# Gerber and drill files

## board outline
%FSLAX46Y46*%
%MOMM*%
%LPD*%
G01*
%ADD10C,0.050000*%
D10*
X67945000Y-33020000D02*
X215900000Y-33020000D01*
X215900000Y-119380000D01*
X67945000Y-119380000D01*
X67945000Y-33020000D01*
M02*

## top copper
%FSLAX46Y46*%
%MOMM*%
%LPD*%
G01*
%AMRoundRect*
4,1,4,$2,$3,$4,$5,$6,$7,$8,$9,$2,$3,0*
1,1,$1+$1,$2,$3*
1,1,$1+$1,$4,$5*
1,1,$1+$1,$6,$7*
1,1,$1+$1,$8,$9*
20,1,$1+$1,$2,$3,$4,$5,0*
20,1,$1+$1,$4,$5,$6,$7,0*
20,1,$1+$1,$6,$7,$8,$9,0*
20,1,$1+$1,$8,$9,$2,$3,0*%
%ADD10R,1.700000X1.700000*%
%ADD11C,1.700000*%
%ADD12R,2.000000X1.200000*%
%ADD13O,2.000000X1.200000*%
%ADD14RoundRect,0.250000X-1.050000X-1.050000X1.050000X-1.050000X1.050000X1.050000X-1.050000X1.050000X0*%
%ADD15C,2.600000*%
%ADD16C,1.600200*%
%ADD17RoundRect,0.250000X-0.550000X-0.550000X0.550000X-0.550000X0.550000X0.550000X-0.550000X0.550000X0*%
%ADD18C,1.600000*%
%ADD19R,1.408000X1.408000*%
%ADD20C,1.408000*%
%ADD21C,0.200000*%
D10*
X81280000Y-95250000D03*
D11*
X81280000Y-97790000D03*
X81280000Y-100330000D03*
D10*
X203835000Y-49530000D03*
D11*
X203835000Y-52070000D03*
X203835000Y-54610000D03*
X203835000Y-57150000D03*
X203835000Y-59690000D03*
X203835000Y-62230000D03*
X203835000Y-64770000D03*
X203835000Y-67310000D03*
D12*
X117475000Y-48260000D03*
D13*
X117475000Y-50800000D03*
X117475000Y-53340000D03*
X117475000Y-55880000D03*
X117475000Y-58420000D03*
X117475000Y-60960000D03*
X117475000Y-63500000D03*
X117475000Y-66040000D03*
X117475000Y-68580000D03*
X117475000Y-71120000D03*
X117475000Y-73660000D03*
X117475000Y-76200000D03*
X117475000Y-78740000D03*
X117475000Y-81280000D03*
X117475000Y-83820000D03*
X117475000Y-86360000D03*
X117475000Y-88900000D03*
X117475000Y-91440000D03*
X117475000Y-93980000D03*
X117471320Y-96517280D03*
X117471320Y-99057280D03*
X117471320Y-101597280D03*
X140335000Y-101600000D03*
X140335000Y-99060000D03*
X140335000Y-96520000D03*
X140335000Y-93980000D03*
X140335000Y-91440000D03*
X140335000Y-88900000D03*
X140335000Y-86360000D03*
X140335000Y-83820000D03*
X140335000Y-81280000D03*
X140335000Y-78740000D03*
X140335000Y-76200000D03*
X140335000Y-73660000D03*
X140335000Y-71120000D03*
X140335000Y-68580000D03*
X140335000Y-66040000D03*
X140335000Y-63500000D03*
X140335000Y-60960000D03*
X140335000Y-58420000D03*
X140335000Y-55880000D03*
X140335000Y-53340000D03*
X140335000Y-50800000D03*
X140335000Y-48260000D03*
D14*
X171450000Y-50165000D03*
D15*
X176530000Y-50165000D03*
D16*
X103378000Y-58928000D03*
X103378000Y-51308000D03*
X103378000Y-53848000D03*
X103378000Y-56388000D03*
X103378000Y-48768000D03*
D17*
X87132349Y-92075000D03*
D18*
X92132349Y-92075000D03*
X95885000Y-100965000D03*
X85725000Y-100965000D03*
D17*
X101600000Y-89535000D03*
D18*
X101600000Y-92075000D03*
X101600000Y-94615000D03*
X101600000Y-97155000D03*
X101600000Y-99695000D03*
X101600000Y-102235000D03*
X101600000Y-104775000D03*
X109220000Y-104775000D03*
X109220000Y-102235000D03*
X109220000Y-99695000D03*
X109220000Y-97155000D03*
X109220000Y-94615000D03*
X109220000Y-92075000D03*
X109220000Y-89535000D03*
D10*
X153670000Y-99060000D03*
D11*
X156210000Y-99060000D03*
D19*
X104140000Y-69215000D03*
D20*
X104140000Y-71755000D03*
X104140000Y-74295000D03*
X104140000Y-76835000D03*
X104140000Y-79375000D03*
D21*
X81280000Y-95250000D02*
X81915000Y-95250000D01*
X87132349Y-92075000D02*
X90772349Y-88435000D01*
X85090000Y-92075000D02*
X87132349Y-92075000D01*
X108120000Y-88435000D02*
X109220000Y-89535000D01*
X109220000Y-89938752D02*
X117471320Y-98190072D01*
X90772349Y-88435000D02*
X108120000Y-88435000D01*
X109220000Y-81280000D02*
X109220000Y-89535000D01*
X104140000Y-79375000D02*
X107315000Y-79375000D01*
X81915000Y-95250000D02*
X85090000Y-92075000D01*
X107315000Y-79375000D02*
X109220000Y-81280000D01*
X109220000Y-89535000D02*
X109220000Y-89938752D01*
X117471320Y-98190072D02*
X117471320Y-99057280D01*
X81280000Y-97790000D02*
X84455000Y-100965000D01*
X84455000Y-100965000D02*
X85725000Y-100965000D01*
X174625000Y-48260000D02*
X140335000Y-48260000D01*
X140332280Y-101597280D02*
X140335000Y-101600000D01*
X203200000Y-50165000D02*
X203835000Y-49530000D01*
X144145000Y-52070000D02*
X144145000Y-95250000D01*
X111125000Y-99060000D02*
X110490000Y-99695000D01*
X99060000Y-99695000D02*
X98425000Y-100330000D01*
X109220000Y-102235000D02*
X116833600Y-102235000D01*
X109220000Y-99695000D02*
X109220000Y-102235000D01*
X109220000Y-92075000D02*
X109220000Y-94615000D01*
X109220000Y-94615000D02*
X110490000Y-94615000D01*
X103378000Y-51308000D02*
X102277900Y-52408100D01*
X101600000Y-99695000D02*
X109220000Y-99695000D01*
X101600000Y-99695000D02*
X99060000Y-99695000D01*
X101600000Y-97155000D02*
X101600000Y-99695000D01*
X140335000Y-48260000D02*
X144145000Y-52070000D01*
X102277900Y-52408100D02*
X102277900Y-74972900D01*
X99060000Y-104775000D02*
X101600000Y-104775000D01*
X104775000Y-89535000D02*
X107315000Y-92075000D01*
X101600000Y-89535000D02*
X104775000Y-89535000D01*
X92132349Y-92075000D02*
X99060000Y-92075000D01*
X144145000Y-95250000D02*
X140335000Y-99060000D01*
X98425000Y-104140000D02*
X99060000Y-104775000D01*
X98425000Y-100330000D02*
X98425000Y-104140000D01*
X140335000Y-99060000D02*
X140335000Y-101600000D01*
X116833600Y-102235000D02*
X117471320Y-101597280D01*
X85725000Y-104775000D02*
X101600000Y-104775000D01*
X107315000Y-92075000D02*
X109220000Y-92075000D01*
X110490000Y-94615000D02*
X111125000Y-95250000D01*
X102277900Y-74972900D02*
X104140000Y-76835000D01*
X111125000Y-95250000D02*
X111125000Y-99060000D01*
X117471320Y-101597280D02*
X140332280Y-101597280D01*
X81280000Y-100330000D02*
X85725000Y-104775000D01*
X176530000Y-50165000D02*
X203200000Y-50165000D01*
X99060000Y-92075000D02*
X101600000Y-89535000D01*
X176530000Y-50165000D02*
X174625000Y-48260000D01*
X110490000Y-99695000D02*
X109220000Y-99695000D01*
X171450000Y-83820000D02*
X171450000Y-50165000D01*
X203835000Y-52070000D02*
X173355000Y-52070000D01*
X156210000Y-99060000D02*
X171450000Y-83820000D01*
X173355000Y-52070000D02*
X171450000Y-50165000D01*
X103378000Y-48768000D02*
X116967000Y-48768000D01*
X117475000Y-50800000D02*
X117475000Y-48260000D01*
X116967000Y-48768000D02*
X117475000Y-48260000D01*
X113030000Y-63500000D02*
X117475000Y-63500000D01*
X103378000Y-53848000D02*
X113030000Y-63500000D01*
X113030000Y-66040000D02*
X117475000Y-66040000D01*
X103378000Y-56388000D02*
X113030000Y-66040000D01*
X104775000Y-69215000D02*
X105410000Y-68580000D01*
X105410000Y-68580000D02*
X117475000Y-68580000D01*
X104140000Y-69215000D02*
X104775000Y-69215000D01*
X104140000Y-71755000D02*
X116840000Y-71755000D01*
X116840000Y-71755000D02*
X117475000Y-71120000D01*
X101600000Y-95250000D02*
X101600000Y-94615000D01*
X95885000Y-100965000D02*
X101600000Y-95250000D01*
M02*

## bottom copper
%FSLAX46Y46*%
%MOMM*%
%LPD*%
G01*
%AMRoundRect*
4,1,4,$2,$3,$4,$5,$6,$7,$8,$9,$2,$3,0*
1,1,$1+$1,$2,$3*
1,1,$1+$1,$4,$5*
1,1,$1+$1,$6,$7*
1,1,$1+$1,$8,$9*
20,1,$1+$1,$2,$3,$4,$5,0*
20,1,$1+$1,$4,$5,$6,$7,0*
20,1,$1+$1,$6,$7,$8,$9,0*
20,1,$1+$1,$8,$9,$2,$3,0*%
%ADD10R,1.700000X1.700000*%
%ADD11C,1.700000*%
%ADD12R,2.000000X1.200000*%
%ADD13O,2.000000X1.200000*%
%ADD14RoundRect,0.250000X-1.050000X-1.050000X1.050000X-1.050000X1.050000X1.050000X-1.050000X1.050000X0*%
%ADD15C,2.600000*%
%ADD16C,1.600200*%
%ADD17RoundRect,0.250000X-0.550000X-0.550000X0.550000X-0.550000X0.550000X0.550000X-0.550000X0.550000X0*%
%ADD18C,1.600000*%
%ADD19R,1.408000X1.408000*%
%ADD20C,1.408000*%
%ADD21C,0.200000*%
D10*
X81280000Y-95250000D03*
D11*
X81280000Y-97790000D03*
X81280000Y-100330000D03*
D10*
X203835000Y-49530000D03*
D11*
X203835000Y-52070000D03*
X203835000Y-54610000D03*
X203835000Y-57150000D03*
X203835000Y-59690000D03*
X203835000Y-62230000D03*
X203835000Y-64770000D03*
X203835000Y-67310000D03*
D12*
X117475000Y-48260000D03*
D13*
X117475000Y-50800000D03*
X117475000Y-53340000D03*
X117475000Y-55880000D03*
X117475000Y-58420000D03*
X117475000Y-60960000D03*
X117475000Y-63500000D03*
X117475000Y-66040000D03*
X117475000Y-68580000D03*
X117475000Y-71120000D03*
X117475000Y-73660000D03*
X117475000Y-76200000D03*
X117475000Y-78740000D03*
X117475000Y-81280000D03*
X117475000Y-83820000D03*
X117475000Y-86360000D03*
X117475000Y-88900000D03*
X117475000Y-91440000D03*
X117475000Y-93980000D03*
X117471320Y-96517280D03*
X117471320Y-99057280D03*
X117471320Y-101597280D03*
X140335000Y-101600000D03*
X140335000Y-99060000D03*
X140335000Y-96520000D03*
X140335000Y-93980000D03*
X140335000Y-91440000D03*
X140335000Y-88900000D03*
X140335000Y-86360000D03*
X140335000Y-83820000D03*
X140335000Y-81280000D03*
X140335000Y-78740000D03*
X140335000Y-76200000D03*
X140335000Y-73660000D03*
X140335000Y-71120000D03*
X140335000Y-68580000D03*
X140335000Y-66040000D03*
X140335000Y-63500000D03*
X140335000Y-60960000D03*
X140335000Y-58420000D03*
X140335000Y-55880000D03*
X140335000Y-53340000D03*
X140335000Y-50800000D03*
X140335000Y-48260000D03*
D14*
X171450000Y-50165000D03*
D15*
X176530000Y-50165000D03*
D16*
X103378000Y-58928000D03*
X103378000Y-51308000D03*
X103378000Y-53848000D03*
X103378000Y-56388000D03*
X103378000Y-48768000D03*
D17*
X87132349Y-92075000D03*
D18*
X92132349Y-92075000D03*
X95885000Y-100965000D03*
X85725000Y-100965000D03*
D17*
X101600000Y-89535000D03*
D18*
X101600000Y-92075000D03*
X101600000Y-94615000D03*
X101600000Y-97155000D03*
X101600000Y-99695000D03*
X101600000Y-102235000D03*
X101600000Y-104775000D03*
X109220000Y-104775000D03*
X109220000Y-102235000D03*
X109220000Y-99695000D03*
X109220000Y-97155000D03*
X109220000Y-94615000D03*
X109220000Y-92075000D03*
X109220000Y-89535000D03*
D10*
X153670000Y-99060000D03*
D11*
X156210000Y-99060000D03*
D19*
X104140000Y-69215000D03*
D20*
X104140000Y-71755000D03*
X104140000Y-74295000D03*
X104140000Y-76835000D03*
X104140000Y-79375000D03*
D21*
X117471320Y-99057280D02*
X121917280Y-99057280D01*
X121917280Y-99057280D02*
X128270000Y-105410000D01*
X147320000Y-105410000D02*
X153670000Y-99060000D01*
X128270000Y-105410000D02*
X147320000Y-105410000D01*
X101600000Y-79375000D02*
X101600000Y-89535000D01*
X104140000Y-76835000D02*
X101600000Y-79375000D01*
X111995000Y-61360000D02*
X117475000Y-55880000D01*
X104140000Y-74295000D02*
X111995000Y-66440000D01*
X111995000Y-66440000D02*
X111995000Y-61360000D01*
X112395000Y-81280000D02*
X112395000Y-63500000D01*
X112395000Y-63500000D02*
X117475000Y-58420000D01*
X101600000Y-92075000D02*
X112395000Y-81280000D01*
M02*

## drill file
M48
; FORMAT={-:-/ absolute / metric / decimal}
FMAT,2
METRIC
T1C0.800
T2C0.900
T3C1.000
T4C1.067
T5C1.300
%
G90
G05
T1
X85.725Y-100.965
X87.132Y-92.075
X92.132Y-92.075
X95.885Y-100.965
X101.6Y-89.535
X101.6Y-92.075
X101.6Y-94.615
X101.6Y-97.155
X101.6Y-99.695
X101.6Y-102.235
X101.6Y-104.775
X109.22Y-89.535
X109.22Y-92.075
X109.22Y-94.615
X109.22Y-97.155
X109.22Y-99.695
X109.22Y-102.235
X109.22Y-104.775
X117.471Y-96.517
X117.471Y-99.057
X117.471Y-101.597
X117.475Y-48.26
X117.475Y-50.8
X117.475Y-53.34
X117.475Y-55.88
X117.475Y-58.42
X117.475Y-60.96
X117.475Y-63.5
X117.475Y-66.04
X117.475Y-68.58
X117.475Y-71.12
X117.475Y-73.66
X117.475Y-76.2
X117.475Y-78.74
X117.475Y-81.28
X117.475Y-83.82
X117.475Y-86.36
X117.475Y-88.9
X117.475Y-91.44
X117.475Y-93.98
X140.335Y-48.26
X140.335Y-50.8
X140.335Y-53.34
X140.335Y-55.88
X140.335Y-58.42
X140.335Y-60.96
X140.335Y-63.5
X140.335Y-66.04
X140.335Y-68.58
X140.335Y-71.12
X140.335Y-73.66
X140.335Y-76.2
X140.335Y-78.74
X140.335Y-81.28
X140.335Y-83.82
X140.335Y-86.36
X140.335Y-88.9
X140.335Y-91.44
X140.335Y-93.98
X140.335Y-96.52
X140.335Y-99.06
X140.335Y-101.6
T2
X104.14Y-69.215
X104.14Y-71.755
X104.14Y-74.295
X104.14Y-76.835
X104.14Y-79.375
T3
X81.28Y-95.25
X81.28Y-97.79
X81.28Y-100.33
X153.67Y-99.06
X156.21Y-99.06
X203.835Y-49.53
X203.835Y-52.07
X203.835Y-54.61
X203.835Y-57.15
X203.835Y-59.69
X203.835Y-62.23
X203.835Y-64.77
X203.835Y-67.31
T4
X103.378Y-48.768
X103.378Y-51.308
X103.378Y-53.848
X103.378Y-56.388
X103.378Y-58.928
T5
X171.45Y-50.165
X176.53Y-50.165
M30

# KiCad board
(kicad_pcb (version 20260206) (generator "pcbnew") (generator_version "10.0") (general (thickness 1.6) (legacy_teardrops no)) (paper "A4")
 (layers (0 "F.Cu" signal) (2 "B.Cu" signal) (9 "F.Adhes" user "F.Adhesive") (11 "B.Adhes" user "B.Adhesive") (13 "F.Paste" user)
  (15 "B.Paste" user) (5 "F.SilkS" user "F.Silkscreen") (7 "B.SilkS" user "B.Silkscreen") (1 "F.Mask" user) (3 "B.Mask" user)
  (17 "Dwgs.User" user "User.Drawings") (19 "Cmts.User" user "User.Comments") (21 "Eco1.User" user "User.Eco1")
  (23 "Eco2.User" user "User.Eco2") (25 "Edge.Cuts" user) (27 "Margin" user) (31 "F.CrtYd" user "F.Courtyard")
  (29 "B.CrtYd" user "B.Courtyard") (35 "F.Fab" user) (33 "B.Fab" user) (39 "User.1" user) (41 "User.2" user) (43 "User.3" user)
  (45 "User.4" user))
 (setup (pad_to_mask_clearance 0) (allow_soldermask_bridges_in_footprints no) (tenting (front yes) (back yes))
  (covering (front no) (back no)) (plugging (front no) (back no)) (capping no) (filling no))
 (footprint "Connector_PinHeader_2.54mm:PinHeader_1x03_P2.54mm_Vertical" (layer "F.Cu") (at 81.28 95.25)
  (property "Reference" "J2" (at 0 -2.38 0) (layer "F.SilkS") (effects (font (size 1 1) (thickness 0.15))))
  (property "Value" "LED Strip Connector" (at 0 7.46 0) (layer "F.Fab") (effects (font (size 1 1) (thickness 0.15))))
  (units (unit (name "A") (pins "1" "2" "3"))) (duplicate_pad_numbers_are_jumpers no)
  (pad "1" thru_hole rect (at 0 0) (size 1.7 1.7) (drill 1) (layers "*.Cu" "*.Mask") (remove_unused_layers no) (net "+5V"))
  (pad "2" thru_hole circle (at 0 2.54) (size 1.7 1.7) (drill 1) (layers "*.Cu" "*.Mask") (remove_unused_layers no) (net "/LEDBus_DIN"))
  (pad "3" thru_hole circle (at 0 5.08) (size 1.7 1.7) (drill 1) (layers "*.Cu" "*.Mask") (remove_unused_layers no) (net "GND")))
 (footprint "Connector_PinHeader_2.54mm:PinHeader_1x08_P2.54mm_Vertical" (layer "F.Cu") (at 203.835 49.53)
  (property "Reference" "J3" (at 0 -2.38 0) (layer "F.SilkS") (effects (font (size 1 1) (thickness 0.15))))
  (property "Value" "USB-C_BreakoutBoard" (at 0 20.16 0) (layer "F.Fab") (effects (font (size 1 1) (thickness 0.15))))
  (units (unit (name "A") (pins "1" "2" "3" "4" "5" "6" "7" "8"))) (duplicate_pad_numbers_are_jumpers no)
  (pad "1" thru_hole rect (at 0 0) (size 1.7 1.7) (drill 1) (layers "*.Cu" "*.Mask") (remove_unused_layers no) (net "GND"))
  (pad "2" thru_hole circle (at 0 2.54) (size 1.7 1.7) (drill 1) (layers "*.Cu" "*.Mask") (remove_unused_layers no) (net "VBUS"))
  (pad "3" thru_hole circle (at 0 5.08) (size 1.7 1.7) (drill 1) (layers "*.Cu" "*.Mask") (remove_unused_layers no)
   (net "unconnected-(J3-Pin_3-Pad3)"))
  (pad "4" thru_hole circle (at 0 7.62) (size 1.7 1.7) (drill 1) (layers "*.Cu" "*.Mask") (remove_unused_layers no)
   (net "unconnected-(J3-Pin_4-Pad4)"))
  (pad "5" thru_hole circle (at 0 10.16) (size 1.7 1.7) (drill 1) (layers "*.Cu" "*.Mask") (remove_unused_layers no)
   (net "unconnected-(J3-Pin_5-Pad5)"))
  (pad "6" thru_hole circle (at 0 12.7) (size 1.7 1.7) (drill 1) (layers "*.Cu" "*.Mask") (remove_unused_layers no)
   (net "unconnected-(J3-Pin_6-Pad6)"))
  (pad "7" thru_hole circle (at 0 15.24) (size 1.7 1.7) (drill 1) (layers "*.Cu" "*.Mask") (remove_unused_layers no)
   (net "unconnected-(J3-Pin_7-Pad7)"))
  (pad "8" thru_hole circle (at 0 17.78) (size 1.7 1.7) (drill 1) (layers "*.Cu" "*.Mask") (remove_unused_layers no)
   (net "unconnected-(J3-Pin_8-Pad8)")))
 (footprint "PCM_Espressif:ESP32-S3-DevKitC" (layer "F.Cu") (at 117.475 48.26)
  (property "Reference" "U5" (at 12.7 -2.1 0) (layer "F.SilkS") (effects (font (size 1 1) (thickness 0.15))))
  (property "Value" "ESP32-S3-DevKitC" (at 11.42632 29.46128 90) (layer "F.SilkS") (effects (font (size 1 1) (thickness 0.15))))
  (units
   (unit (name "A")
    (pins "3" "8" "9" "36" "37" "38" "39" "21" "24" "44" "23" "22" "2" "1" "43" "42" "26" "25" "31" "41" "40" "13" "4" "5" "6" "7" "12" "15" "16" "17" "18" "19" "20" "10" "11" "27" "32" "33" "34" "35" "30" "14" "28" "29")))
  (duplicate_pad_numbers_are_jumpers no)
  (pad "1" thru_hole rect (at 0 0 270) (size 1.2 2) (drill 0.8) (layers "*.Cu" "*.Mask") (remove_unused_layers no) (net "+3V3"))
  (pad "2" thru_hole oval (at 0 2.54 270) (size 1.2 2) (drill 0.8) (layers "*.Cu" "*.Mask") (remove_unused_layers no) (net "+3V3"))
  (pad "3" thru_hole oval (at 0 5.08 270) (size 1.2 2) (drill 0.8) (layers "*.Cu" "*.Mask") (remove_unused_layers no)
   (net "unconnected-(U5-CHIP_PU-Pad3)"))
  (pad "4" thru_hole oval (at 0 7.62 270) (size 1.2 2) (drill 0.8) (layers "*.Cu" "*.Mask") (remove_unused_layers no)
   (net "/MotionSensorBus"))
  (pad "5" thru_hole oval (at 0 10.16 270) (size 1.2 2) (drill 0.8) (layers "*.Cu" "*.Mask") (remove_unused_layers no) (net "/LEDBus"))
  (pad "6" thru_hole oval (at 0 12.7 270) (size 1.2 2) (drill 0.8) (layers "*.Cu" "*.Mask") (remove_unused_layers no)
   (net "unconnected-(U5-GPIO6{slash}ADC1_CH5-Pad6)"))
  (pad "7" thru_hole oval (at 0 15.24 270) (size 1.2 2) (drill 0.8) (layers "*.Cu" "*.Mask") (remove_unused_layers no) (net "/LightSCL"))
  (pad "8" thru_hole oval (at 0 17.78 270) (size 1.2 2) (drill 0.8) (layers "*.Cu" "*.Mask") (remove_unused_layers no) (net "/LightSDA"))
  (pad "9" thru_hole oval (at 0 20.32 270) (size 1.2 2) (drill 0.8) (layers "*.Cu" "*.Mask") (remove_unused_layers no)
   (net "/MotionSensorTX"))
  (pad "10" thru_hole oval (at 0 22.86 270) (size 1.2 2) (drill 0.8) (layers "*.Cu" "*.Mask") (remove_unused_layers no)
   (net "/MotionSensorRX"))
  (pad "11" thru_hole oval (at 0 25.4 270) (size 1.2 2) (drill 0.8) (layers "*.Cu" "*.Mask") (remove_unused_layers no)
   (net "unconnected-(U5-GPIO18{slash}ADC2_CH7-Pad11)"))
  (pad "12" thru_hole oval (at 0 27.94 270) (size 1.2 2) (drill 0.8) (layers "*.Cu" "*.Mask") (remove_unused_layers no)
   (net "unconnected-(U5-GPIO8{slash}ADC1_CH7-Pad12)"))
  (pad "13" thru_hole oval (at 0 30.48 270) (size 1.2 2) (drill 0.8) (layers "*.Cu" "*.Mask") (remove_unused_layers no)
   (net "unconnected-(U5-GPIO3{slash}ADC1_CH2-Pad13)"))
  (pad "14" thru_hole oval (at 0 33.02 270) (size 1.2 2) (drill 0.8) (layers "*.Cu" "*.Mask") (remove_unused_layers no)
   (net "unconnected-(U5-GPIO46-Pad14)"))
  (pad "15" thru_hole oval (at 0 35.56 270) (size 1.2 2) (drill 0.8) (layers "*.Cu" "*.Mask") (remove_unused_layers no)
   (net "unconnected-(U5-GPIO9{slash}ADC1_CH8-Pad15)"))
  (pad "16" thru_hole oval (at 0 38.1 270) (size 1.2 2) (drill 0.8) (layers "*.Cu" "*.Mask") (remove_unused_layers no)
   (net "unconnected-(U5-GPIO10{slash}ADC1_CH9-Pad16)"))
  (pad "17" thru_hole oval (at 0 40.64 270) (size 1.2 2) (drill 0.8) (layers "*.Cu" "*.Mask") (remove_unused_layers no)
   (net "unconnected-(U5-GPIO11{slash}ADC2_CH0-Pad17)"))
  (pad "18" thru_hole oval (at 0 43.18 270) (size 1.2 2) (drill 0.8) (layers "*.Cu" "*.Mask") (remove_unused_layers no)
   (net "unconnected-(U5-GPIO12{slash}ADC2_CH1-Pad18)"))
  (pad "19" thru_hole oval (at 0 45.72 270) (size 1.2 2) (drill 0.8) (layers "*.Cu" "*.Mask") (remove_unused_layers no)
   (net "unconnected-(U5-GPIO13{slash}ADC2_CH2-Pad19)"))
  (pad "20" thru_hole oval (at -0.00368 48.25728 270) (size 1.2 2) (drill 0.8) (layers "*.Cu" "*.Mask") (remove_unused_layers no)
   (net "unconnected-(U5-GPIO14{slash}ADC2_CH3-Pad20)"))
  (pad "21" thru_hole oval (at -0.00368 50.79728 270) (size 1.2 2) (drill 0.8) (layers "*.Cu" "*.Mask") (remove_unused_layers no)
   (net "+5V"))
  (pad "22" thru_hole oval (at -0.00368 53.33728 270) (size 1.2 2) (drill 0.8) (layers "*.Cu" "*.Mask") (remove_unused_layers no)
   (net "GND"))
  (pad "23" thru_hole oval (at 22.86 53.34 270) (size 1.2 2) (drill 0.8) (layers "*.Cu" "*.Mask") (remove_unused_layers no) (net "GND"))
  (pad "24" thru_hole oval (at 22.86 50.8 270) (size 1.2 2) (drill 0.8) (layers "*.Cu" "*.Mask") (remove_unused_layers no) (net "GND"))
  (pad "25" thru_hole oval (at 22.86 48.26 270) (size 1.2 2) (drill 0.8) (layers "*.Cu" "*.Mask") (remove_unused_layers no)
   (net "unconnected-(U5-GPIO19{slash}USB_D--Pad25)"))
  (pad "26" thru_hole oval (at 22.86 45.72 270) (size 1.2 2) (drill 0.8) (layers "*.Cu" "*.Mask") (remove_unused_layers no)
   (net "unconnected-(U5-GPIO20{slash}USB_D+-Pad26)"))
  (pad "27" thru_hole oval (at 22.86 43.18 270) (size 1.2 2) (drill 0.8) (layers "*.Cu" "*.Mask") (remove_unused_layers no)
   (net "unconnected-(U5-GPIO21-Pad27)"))
  (pad "28" thru_hole oval (at 22.86 40.64 270) (size 1.2 2) (drill 0.8) (layers "*.Cu" "*.Mask") (remove_unused_layers no)
   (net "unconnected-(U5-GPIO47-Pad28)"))
  (pad "29" thru_hole oval (at 22.86 38.1 270) (size 1.2 2) (drill 0.8) (layers "*.Cu" "*.Mask") (remove_unused_layers no)
   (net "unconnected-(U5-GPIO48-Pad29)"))
  (pad "30" thru_hole oval (at 22.86 35.56 270) (size 1.2 2) (drill 0.8) (layers "*.Cu" "*.Mask") (remove_unused_layers no)
   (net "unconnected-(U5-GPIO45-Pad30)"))
  (pad "31" thru_hole oval (at 22.86 33.02 270) (size 1.2 2) (drill 0.8) (layers "*.Cu" "*.Mask") (remove_unused_layers no)
   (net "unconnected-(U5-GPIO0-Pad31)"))
  (pad "32" thru_hole oval (at 22.86 30.48 270) (size 1.2 2) (drill 0.8) (layers "*.Cu" "*.Mask") (remove_unused_layers no)
   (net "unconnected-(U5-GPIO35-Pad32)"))
  (pad "33" thru_hole oval (at 22.86 27.94 270) (size 1.2 2) (drill 0.8) (layers "*.Cu" "*.Mask") (remove_unused_layers no)
   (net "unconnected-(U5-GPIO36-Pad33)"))
  (pad "34" thru_hole oval (at 22.86 25.4 270) (size 1.2 2) (drill 0.8) (layers "*.Cu" "*.Mask") (remove_unused_layers no)
   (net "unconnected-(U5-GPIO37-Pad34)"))
  (pad "35" thru_hole oval (at 22.86 22.86 270) (size 1.2 2) (drill 0.8) (layers "*.Cu" "*.Mask") (remove_unused_layers no)
   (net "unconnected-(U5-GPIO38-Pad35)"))
  (pad "36" thru_hole oval (at 22.86 20.32 270) (size 1.2 2) (drill 0.8) (layers "*.Cu" "*.Mask") (remove_unused_layers no)
   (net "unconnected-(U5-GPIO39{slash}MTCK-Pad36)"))
  (pad "37" thru_hole oval (at 22.86 17.78 270) (size 1.2 2) (drill 0.8) (layers "*.Cu" "*.Mask") (remove_unused_layers no)
   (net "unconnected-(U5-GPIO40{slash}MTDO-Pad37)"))
  (pad "38" thru_hole oval (at 22.86 15.24 270) (size 1.2 2) (drill 0.8) (layers "*.Cu" "*.Mask") (remove_unused_layers no)
   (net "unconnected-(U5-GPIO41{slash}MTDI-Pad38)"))
  (pad "39" thru_hole oval (at 22.86 12.7 270) (size 1.2 2) (drill 0.8) (layers "*.Cu" "*.Mask") (remove_unused_layers no)
   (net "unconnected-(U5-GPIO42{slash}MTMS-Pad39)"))
  (pad "40" thru_hole oval (at 22.86 10.16 270) (size 1.2 2) (drill 0.8) (layers "*.Cu" "*.Mask") (remove_unused_layers no)
   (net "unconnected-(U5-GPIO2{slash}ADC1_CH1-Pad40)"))
  (pad "41" thru_hole oval (at 22.86 7.62 270) (size 1.2 2) (drill 0.8) (layers "*.Cu" "*.Mask") (remove_unused_layers no)
   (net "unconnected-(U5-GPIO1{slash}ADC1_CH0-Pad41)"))
  (pad "42" thru_hole oval (at 22.86 5.08 270) (size 1.2 2) (drill 0.8) (layers "*.Cu" "*.Mask") (remove_unused_layers no)
   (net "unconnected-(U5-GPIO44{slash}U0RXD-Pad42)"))
  (pad "43" thru_hole oval (at 22.86 2.54 270) (size 1.2 2) (drill 0.8) (layers "*.Cu" "*.Mask") (remove_unused_layers no)
   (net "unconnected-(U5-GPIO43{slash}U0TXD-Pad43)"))
  (pad "44" thru_hole oval (at 22.86 0 270) (size 1.2 2) (drill 0.8) (layers "*.Cu" "*.Mask") (remove_unused_layers no) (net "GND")))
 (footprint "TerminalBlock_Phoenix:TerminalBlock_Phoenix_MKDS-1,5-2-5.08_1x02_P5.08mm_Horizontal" (layer "F.Cu") (at 171.45 50.165)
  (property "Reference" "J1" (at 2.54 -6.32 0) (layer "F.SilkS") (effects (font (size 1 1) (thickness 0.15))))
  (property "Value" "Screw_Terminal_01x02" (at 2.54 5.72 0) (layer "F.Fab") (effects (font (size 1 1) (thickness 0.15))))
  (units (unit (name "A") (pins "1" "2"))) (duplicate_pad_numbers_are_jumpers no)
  (pad "1" thru_hole roundrect (at 0 0) (size 2.6 2.6) (drill 1.3) (layers "*.Cu" "*.Mask") (remove_unused_layers no)
   (roundrect_rratio 0.096154) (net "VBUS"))
  (pad "2" thru_hole circle (at 5.08 0) (size 2.6 2.6) (drill 1.3) (layers "*.Cu" "*.Mask") (remove_unused_layers no) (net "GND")))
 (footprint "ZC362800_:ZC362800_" (layer "F.Cu") (at 102.108 53.848 -90)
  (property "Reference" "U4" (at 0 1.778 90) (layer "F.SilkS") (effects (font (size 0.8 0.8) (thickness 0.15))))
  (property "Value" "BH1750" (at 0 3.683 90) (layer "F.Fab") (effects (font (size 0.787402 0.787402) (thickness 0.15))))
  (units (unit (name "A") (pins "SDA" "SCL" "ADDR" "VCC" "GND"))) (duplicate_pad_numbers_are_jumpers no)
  (pad "ADDR" thru_hole circle (at 5.08 -1.27 270) (size 1.6002 1.6002) (drill 1.0668) (layers "*.Cu" "*.Mask") (remove_unused_layers no)
   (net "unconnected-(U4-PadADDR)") (solder_mask_margin 0.102))
  (pad "GND" thru_hole circle (at -2.54 -1.27 270) (size 1.6002 1.6002) (drill 1.0668) (layers "*.Cu" "*.Mask") (remove_unused_layers no)
   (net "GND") (solder_mask_margin 0.102))
  (pad "SCL" thru_hole circle (at 0 -1.27 270) (size 1.6002 1.6002) (drill 1.0668) (layers "*.Cu" "*.Mask") (remove_unused_layers no)
   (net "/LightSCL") (solder_mask_margin 0.102))
  (pad "SDA" thru_hole circle (at 2.54 -1.27 270) (size 1.6002 1.6002) (drill 1.0668) (layers "*.Cu" "*.Mask") (remove_unused_layers no)
   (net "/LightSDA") (solder_mask_margin 0.102))
  (pad "VCC" thru_hole circle (at -5.08 -1.27 270) (size 1.6002 1.6002) (drill 1.0668) (layers "*.Cu" "*.Mask") (remove_unused_layers no)
   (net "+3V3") (solder_mask_margin 0.102)))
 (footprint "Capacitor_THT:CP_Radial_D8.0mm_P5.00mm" (layer "F.Cu") (at 87.132349 92.075)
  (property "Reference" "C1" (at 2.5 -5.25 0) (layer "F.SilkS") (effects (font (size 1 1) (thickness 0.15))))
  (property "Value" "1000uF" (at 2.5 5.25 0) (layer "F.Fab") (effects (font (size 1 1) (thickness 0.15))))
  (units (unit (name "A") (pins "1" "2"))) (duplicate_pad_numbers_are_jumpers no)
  (pad "1" thru_hole roundrect (at 0 0) (size 1.6 1.6) (drill 0.8) (layers "*.Cu" "*.Mask") (remove_unused_layers no)
   (roundrect_rratio 0.15625) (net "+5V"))
  (pad "2" thru_hole circle (at 5 0) (size 1.6 1.6) (drill 0.8) (layers "*.Cu" "*.Mask") (remove_unused_layers no) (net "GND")))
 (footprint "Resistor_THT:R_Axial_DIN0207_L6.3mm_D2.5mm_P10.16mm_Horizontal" (layer "F.Cu") (at 95.885 100.965 180)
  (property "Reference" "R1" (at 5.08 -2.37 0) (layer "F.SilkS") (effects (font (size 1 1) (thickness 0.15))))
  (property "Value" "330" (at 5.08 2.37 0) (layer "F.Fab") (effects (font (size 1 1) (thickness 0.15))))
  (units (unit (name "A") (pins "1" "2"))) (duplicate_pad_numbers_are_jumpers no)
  (pad "1" thru_hole circle (at 0 0 180) (size 1.6 1.6) (drill 0.8) (layers "*.Cu" "*.Mask") (remove_unused_layers no) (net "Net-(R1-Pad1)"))
  (pad "2" thru_hole circle (at 10.16 0 180) (size 1.6 1.6) (drill 0.8) (layers "*.Cu" "*.Mask") (remove_unused_layers no)
   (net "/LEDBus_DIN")))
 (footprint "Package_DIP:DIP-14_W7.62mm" (layer "F.Cu") (at 101.6 89.535)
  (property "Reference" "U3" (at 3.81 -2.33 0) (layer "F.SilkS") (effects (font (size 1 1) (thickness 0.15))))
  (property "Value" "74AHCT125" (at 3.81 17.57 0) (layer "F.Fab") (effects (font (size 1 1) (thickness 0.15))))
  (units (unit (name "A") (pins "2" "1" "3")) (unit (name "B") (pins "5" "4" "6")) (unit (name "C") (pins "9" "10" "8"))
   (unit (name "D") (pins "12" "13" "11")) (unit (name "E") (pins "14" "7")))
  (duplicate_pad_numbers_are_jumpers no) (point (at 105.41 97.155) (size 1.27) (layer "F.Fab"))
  (pad "1" thru_hole roundrect (at 0 0) (size 1.6 1.6) (drill 0.8) (layers "*.Cu" "*.Mask") (remove_unused_layers no)
   (roundrect_rratio 0.15625) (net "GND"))
  (pad "2" thru_hole circle (at 0 2.54) (size 1.6 1.6) (drill 0.8) (layers "*.Cu" "*.Mask") (remove_unused_layers no) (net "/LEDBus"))
  (pad "3" thru_hole circle (at 0 5.08) (size 1.6 1.6) (drill 0.8) (layers "*.Cu" "*.Mask") (remove_unused_layers no) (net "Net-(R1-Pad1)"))
  (pad "4" thru_hole circle (at 0 7.62) (size 1.6 1.6) (drill 0.8) (layers "*.Cu" "*.Mask") (remove_unused_layers no) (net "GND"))
  (pad "5" thru_hole circle (at 0 10.16) (size 1.6 1.6) (drill 0.8) (layers "*.Cu" "*.Mask") (remove_unused_layers no) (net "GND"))
  (pad "6" thru_hole circle (at 0 12.7) (size 1.6 1.6) (drill 0.8) (layers "*.Cu" "*.Mask") (remove_unused_layers no)
   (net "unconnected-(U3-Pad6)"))
  (pad "7" thru_hole circle (at 0 15.24) (size 1.6 1.6) (drill 0.8) (layers "*.Cu" "*.Mask") (remove_unused_layers no) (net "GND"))
  (pad "8" thru_hole circle (at 7.62 15.24) (size 1.6 1.6) (drill 0.8) (layers "*.Cu" "*.Mask") (remove_unused_layers no)
   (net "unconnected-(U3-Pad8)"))
  (pad "9" thru_hole circle (at 7.62 12.7) (size 1.6 1.6) (drill 0.8) (layers "*.Cu" "*.Mask") (remove_unused_layers no) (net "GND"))
  (pad "10" thru_hole circle (at 7.62 10.16) (size 1.6 1.6) (drill 0.8) (layers "*.Cu" "*.Mask") (remove_unused_layers no) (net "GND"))
  (pad "11" thru_hole circle (at 7.62 7.62) (size 1.6 1.6) (drill 0.8) (layers "*.Cu" "*.Mask") (remove_unused_layers no)
   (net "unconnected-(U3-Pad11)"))
  (pad "12" thru_hole circle (at 7.62 5.08) (size 1.6 1.6) (drill 0.8) (layers "*.Cu" "*.Mask") (remove_unused_layers no) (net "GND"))
  (pad "13" thru_hole circle (at 7.62 2.54) (size 1.6 1.6) (drill 0.8) (layers "*.Cu" "*.Mask") (remove_unused_layers no) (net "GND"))
  (pad "14" thru_hole circle (at 7.62 0) (size 1.6 1.6) (drill 0.8) (layers "*.Cu" "*.Mask") (remove_unused_layers no) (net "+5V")))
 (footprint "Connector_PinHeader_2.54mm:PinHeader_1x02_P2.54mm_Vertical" (layer "F.Cu") (at 153.67 99.06 90)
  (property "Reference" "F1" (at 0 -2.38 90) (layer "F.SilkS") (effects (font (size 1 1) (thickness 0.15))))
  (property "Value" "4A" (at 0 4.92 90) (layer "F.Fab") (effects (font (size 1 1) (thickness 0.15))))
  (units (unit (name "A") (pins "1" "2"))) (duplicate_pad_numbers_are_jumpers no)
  (pad "1" thru_hole rect (at 0 0 90) (size 1.7 1.7) (drill 1) (layers "*.Cu" "*.Mask") (remove_unused_layers no) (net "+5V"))
  (pad "2" thru_hole circle (at 0 2.54 90) (size 1.7 1.7) (drill 1) (layers "*.Cu" "*.Mask") (remove_unused_layers no) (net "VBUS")))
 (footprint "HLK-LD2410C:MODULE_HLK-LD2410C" (layer "F.Cu") (at 97.6 74.245 -90)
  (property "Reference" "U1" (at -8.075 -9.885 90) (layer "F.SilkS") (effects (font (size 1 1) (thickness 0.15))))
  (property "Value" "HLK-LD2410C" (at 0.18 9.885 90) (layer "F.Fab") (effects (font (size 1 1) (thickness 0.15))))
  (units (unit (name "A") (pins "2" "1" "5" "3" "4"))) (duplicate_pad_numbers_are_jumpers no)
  (pad "1" thru_hole rect (at -5.03 -6.54 270) (size 1.408 1.408) (drill 0.9) (layers "*.Cu" "*.Mask") (remove_unused_layers no)
   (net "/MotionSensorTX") (solder_mask_margin 0.102))
  (pad "2" thru_hole circle (at -2.49 -6.54 270) (size 1.408 1.408) (drill 0.9) (layers "*.Cu" "*.Mask") (remove_unused_layers no)
   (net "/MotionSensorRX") (solder_mask_margin 0.102))
  (pad "3" thru_hole circle (at 0.05 -6.54 270) (size 1.408 1.408) (drill 0.9) (layers "*.Cu" "*.Mask") (remove_unused_layers no)
   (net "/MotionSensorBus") (solder_mask_margin 0.102))
  (pad "4" thru_hole circle (at 2.59 -6.54 270) (size 1.408 1.408) (drill 0.9) (layers "*.Cu" "*.Mask") (remove_unused_layers no)
   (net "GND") (solder_mask_margin 0.102))
  (pad "5" thru_hole circle (at 5.13 -6.54 270) (size 1.408 1.408) (drill 0.9) (layers "*.Cu" "*.Mask") (remove_unused_layers no)
   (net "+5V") (solder_mask_margin 0.102)))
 (gr_rect (start 67.945 33.02) (end 215.9 119.38) (stroke (width 0.05) (type default)) (fill no) (layer "Edge.Cuts"))
 (segment (start 81.28 95.25) (end 81.915 95.25) (width 0.2) (layer "F.Cu") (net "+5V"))
 (segment (start 87.132349 92.075) (end 90.772349 88.435) (width 0.2) (layer "F.Cu") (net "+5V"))
 (segment (start 85.09 92.075) (end 87.132349 92.075) (width 0.2) (layer "F.Cu") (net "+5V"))
 (segment (start 108.12 88.435) (end 109.22 89.535) (width 0.2) (layer "F.Cu") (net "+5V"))
 (segment (start 109.22 89.938752) (end 117.47132 98.190072) (width 0.2) (layer "F.Cu") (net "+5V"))
 (segment (start 90.772349 88.435) (end 108.12 88.435) (width 0.2) (layer "F.Cu") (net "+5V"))
 (segment (start 109.22 81.28) (end 109.22 89.535) (width 0.2) (layer "F.Cu") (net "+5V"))
 (segment (start 104.14 79.375) (end 107.315 79.375) (width 0.2) (layer "F.Cu") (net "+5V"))
 (segment (start 81.915 95.25) (end 85.09 92.075) (width 0.2) (layer "F.Cu") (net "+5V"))
 (segment (start 107.315 79.375) (end 109.22 81.28) (width 0.2) (layer "F.Cu") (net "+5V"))
 (segment (start 109.22 89.535) (end 109.22 89.938752) (width 0.2) (layer "F.Cu") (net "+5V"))
 (segment (start 117.47132 98.190072) (end 117.47132 99.05728) (width 0.2) (layer "F.Cu") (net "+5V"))
 (segment (start 117.47132 99.05728) (end 121.91728 99.05728) (width 0.2) (layer "B.Cu") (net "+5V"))
 (segment (start 121.91728 99.05728) (end 128.27 105.41) (width 0.2) (layer "B.Cu") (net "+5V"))
 (segment (start 147.32 105.41) (end 153.67 99.06) (width 0.2) (layer "B.Cu") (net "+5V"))
 (segment (start 128.27 105.41) (end 147.32 105.41) (width 0.2) (layer "B.Cu") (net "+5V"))
 (segment (start 81.28 97.79) (end 84.455 100.965) (width 0.2) (layer "F.Cu") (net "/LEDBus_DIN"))
 (segment (start 84.455 100.965) (end 85.725 100.965) (width 0.2) (layer "F.Cu") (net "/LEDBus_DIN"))
 (segment (start 174.625 48.26) (end 140.335 48.26) (width 0.2) (layer "F.Cu") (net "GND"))
 (segment (start 140.33228 101.59728) (end 140.335 101.6) (width 0.2) (layer "F.Cu") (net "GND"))
 (segment (start 203.2 50.165) (end 203.835 49.53) (width 0.2) (layer "F.Cu") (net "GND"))
 (segment (start 144.145 52.07) (end 144.145 95.25) (width 0.2) (layer "F.Cu") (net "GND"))
 (segment (start 111.125 99.06) (end 110.49 99.695) (width 0.2) (layer "F.Cu") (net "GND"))
 (segment (start 99.06 99.695) (end 98.425 100.33) (width 0.2) (layer "F.Cu") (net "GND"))
 (segment (start 109.22 102.235) (end 116.8336 102.235) (width 0.2) (layer "F.Cu") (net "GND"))
 (segment (start 109.22 99.695) (end 109.22 102.235) (width 0.2) (layer "F.Cu") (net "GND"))
 (segment (start 109.22 92.075) (end 109.22 94.615) (width 0.2) (layer "F.Cu") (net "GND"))
 (segment (start 109.22 94.615) (end 110.49 94.615) (width 0.2) (layer "F.Cu") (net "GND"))
 (segment (start 103.378 51.308) (end 102.2779 52.4081) (width 0.2) (layer "F.Cu") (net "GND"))
 (segment (start 101.6 99.695) (end 109.22 99.695) (width 0.2) (layer "F.Cu") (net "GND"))
 (segment (start 101.6 99.695) (end 99.06 99.695) (width 0.2) (layer "F.Cu") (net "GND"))
 (segment (start 101.6 97.155) (end 101.6 99.695) (width 0.2) (layer "F.Cu") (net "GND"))
 (segment (start 140.335 48.26) (end 144.145 52.07) (width 0.2) (layer "F.Cu") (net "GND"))
 (segment (start 102.2779 52.4081) (end 102.2779 74.9729) (width 0.2) (layer "F.Cu") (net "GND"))
 (segment (start 99.06 104.775) (end 101.6 104.775) (width 0.2) (layer "F.Cu") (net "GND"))
 (segment (start 104.775 89.535) (end 107.315 92.075) (width 0.2) (layer "F.Cu") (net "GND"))
 (segment (start 101.6 89.535) (end 104.775 89.535) (width 0.2) (layer "F.Cu") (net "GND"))
 (segment (start 92.132349 92.075) (end 99.06 92.075) (width 0.2) (layer "F.Cu") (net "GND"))
 (segment (start 144.145 95.25) (end 140.335 99.06) (width 0.2) (layer "F.Cu") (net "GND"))
 (segment (start 98.425 104.14) (end 99.06 104.775) (width 0.2) (layer "F.Cu") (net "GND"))
 (segment (start 98.425 100.33) (end 98.425 104.14) (width 0.2) (layer "F.Cu") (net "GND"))
 (segment (start 140.335 99.06) (end 140.335 101.6) (width 0.2) (layer "F.Cu") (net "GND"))
 (segment (start 116.8336 102.235) (end 117.47132 101.59728) (width 0.2) (layer "F.Cu") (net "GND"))
 (segment (start 85.725 104.775) (end 101.6 104.775) (width 0.2) (layer "F.Cu") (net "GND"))
 (segment (start 107.315 92.075) (end 109.22 92.075) (width 0.2) (layer "F.Cu") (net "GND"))
 (segment (start 110.49 94.615) (end 111.125 95.25) (width 0.2) (layer "F.Cu") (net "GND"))
 (segment (start 102.2779 74.9729) (end 104.14 76.835) (width 0.2) (layer "F.Cu") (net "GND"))
 (segment (start 111.125 95.25) (end 111.125 99.06) (width 0.2) (layer "F.Cu") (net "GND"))
 (segment (start 117.47132 101.59728) (end 140.33228 101.59728) (width 0.2) (layer "F.Cu") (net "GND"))
 (segment (start 81.28 100.33) (end 85.725 104.775) (width 0.2) (layer "F.Cu") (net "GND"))
 (segment (start 176.53 50.165) (end 203.2 50.165) (width 0.2) (layer "F.Cu") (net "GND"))
 (segment (start 99.06 92.075) (end 101.6 89.535) (width 0.2) (layer "F.Cu") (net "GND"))
 (segment (start 176.53 50.165) (end 174.625 48.26) (width 0.2) (layer "F.Cu") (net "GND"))
 (segment (start 110.49 99.695) (end 109.22 99.695) (width 0.2) (layer "F.Cu") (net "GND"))
 (segment (start 101.6 79.375) (end 101.6 89.535) (width 0.2) (layer "B.Cu") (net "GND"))
 (segment (start 104.14 76.835) (end 101.6 79.375) (width 0.2) (layer "B.Cu") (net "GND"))
 (segment (start 171.45 83.82) (end 171.45 50.165) (width 0.2) (layer "F.Cu") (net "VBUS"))
 (segment (start 203.835 52.07) (end 173.355 52.07) (width 0.2) (layer "F.Cu") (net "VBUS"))
 (segment (start 156.21 99.06) (end 171.45 83.82) (width 0.2) (layer "F.Cu") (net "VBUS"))
 (segment (start 173.355 52.07) (end 171.45 50.165) (width 0.2) (layer "F.Cu") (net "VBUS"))
 (segment (start 103.378 48.768) (end 116.967 48.768) (width 0.2) (layer "F.Cu") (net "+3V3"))
 (segment (start 117.475 50.8) (end 117.475 48.26) (width 0.2) (layer "F.Cu") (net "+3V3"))
 (segment (start 116.967 48.768) (end 117.475 48.26) (width 0.2) (layer "F.Cu") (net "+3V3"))
 (segment (start 111.995 61.36) (end 117.475 55.88) (width 0.2) (layer "B.Cu") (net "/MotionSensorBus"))
 (segment (start 104.14 74.295) (end 111.995 66.44) (width 0.2) (layer "B.Cu") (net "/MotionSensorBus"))
 (segment (start 111.995 66.44) (end 111.995 61.36) (width 0.2) (layer "B.Cu") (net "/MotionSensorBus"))
 (segment (start 112.395 81.28) (end 112.395 63.5) (width 0.2) (layer "B.Cu") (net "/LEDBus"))
 (segment (start 112.395 63.5) (end 117.475 58.42) (width 0.2) (layer "B.Cu") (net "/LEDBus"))
 (segment (start 101.6 92.075) (end 112.395 81.28) (width 0.2) (layer "B.Cu") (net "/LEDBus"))
 (segment (start 113.03 63.5) (end 117.475 63.5) (width 0.2) (layer "F.Cu") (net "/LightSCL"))
 (segment (start 103.378 53.848) (end 113.03 63.5) (width 0.2) (layer "F.Cu") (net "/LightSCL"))
 (segment (start 113.03 66.04) (end 117.475 66.04) (width 0.2) (layer "F.Cu") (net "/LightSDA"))
 (segment (start 103.378 56.388) (end 113.03 66.04) (width 0.2) (layer "F.Cu") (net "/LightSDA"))
 (segment (start 104.775 69.215) (end 105.41 68.58) (width 0.2) (layer "F.Cu") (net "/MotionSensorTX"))
 (segment (start 105.41 68.58) (end 117.475 68.58) (width 0.2) (layer "F.Cu") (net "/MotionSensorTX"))
 (segment (start 104.14 69.215) (end 104.775 69.215) (width 0.2) (layer "F.Cu") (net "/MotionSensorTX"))
 (segment (start 104.14 71.755) (end 116.84 71.755) (width 0.2) (layer "F.Cu") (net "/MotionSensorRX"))
 (segment (start 116.84 71.755) (end 117.475 71.12) (width 0.2) (layer "F.Cu") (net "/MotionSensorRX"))
 (segment (start 101.6 95.25) (end 101.6 94.615) (width 0.2) (layer "F.Cu") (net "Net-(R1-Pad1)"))
 (segment (start 95.885 100.965) (end 101.6 95.25) (width 0.2) (layer "F.Cu") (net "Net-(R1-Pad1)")))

